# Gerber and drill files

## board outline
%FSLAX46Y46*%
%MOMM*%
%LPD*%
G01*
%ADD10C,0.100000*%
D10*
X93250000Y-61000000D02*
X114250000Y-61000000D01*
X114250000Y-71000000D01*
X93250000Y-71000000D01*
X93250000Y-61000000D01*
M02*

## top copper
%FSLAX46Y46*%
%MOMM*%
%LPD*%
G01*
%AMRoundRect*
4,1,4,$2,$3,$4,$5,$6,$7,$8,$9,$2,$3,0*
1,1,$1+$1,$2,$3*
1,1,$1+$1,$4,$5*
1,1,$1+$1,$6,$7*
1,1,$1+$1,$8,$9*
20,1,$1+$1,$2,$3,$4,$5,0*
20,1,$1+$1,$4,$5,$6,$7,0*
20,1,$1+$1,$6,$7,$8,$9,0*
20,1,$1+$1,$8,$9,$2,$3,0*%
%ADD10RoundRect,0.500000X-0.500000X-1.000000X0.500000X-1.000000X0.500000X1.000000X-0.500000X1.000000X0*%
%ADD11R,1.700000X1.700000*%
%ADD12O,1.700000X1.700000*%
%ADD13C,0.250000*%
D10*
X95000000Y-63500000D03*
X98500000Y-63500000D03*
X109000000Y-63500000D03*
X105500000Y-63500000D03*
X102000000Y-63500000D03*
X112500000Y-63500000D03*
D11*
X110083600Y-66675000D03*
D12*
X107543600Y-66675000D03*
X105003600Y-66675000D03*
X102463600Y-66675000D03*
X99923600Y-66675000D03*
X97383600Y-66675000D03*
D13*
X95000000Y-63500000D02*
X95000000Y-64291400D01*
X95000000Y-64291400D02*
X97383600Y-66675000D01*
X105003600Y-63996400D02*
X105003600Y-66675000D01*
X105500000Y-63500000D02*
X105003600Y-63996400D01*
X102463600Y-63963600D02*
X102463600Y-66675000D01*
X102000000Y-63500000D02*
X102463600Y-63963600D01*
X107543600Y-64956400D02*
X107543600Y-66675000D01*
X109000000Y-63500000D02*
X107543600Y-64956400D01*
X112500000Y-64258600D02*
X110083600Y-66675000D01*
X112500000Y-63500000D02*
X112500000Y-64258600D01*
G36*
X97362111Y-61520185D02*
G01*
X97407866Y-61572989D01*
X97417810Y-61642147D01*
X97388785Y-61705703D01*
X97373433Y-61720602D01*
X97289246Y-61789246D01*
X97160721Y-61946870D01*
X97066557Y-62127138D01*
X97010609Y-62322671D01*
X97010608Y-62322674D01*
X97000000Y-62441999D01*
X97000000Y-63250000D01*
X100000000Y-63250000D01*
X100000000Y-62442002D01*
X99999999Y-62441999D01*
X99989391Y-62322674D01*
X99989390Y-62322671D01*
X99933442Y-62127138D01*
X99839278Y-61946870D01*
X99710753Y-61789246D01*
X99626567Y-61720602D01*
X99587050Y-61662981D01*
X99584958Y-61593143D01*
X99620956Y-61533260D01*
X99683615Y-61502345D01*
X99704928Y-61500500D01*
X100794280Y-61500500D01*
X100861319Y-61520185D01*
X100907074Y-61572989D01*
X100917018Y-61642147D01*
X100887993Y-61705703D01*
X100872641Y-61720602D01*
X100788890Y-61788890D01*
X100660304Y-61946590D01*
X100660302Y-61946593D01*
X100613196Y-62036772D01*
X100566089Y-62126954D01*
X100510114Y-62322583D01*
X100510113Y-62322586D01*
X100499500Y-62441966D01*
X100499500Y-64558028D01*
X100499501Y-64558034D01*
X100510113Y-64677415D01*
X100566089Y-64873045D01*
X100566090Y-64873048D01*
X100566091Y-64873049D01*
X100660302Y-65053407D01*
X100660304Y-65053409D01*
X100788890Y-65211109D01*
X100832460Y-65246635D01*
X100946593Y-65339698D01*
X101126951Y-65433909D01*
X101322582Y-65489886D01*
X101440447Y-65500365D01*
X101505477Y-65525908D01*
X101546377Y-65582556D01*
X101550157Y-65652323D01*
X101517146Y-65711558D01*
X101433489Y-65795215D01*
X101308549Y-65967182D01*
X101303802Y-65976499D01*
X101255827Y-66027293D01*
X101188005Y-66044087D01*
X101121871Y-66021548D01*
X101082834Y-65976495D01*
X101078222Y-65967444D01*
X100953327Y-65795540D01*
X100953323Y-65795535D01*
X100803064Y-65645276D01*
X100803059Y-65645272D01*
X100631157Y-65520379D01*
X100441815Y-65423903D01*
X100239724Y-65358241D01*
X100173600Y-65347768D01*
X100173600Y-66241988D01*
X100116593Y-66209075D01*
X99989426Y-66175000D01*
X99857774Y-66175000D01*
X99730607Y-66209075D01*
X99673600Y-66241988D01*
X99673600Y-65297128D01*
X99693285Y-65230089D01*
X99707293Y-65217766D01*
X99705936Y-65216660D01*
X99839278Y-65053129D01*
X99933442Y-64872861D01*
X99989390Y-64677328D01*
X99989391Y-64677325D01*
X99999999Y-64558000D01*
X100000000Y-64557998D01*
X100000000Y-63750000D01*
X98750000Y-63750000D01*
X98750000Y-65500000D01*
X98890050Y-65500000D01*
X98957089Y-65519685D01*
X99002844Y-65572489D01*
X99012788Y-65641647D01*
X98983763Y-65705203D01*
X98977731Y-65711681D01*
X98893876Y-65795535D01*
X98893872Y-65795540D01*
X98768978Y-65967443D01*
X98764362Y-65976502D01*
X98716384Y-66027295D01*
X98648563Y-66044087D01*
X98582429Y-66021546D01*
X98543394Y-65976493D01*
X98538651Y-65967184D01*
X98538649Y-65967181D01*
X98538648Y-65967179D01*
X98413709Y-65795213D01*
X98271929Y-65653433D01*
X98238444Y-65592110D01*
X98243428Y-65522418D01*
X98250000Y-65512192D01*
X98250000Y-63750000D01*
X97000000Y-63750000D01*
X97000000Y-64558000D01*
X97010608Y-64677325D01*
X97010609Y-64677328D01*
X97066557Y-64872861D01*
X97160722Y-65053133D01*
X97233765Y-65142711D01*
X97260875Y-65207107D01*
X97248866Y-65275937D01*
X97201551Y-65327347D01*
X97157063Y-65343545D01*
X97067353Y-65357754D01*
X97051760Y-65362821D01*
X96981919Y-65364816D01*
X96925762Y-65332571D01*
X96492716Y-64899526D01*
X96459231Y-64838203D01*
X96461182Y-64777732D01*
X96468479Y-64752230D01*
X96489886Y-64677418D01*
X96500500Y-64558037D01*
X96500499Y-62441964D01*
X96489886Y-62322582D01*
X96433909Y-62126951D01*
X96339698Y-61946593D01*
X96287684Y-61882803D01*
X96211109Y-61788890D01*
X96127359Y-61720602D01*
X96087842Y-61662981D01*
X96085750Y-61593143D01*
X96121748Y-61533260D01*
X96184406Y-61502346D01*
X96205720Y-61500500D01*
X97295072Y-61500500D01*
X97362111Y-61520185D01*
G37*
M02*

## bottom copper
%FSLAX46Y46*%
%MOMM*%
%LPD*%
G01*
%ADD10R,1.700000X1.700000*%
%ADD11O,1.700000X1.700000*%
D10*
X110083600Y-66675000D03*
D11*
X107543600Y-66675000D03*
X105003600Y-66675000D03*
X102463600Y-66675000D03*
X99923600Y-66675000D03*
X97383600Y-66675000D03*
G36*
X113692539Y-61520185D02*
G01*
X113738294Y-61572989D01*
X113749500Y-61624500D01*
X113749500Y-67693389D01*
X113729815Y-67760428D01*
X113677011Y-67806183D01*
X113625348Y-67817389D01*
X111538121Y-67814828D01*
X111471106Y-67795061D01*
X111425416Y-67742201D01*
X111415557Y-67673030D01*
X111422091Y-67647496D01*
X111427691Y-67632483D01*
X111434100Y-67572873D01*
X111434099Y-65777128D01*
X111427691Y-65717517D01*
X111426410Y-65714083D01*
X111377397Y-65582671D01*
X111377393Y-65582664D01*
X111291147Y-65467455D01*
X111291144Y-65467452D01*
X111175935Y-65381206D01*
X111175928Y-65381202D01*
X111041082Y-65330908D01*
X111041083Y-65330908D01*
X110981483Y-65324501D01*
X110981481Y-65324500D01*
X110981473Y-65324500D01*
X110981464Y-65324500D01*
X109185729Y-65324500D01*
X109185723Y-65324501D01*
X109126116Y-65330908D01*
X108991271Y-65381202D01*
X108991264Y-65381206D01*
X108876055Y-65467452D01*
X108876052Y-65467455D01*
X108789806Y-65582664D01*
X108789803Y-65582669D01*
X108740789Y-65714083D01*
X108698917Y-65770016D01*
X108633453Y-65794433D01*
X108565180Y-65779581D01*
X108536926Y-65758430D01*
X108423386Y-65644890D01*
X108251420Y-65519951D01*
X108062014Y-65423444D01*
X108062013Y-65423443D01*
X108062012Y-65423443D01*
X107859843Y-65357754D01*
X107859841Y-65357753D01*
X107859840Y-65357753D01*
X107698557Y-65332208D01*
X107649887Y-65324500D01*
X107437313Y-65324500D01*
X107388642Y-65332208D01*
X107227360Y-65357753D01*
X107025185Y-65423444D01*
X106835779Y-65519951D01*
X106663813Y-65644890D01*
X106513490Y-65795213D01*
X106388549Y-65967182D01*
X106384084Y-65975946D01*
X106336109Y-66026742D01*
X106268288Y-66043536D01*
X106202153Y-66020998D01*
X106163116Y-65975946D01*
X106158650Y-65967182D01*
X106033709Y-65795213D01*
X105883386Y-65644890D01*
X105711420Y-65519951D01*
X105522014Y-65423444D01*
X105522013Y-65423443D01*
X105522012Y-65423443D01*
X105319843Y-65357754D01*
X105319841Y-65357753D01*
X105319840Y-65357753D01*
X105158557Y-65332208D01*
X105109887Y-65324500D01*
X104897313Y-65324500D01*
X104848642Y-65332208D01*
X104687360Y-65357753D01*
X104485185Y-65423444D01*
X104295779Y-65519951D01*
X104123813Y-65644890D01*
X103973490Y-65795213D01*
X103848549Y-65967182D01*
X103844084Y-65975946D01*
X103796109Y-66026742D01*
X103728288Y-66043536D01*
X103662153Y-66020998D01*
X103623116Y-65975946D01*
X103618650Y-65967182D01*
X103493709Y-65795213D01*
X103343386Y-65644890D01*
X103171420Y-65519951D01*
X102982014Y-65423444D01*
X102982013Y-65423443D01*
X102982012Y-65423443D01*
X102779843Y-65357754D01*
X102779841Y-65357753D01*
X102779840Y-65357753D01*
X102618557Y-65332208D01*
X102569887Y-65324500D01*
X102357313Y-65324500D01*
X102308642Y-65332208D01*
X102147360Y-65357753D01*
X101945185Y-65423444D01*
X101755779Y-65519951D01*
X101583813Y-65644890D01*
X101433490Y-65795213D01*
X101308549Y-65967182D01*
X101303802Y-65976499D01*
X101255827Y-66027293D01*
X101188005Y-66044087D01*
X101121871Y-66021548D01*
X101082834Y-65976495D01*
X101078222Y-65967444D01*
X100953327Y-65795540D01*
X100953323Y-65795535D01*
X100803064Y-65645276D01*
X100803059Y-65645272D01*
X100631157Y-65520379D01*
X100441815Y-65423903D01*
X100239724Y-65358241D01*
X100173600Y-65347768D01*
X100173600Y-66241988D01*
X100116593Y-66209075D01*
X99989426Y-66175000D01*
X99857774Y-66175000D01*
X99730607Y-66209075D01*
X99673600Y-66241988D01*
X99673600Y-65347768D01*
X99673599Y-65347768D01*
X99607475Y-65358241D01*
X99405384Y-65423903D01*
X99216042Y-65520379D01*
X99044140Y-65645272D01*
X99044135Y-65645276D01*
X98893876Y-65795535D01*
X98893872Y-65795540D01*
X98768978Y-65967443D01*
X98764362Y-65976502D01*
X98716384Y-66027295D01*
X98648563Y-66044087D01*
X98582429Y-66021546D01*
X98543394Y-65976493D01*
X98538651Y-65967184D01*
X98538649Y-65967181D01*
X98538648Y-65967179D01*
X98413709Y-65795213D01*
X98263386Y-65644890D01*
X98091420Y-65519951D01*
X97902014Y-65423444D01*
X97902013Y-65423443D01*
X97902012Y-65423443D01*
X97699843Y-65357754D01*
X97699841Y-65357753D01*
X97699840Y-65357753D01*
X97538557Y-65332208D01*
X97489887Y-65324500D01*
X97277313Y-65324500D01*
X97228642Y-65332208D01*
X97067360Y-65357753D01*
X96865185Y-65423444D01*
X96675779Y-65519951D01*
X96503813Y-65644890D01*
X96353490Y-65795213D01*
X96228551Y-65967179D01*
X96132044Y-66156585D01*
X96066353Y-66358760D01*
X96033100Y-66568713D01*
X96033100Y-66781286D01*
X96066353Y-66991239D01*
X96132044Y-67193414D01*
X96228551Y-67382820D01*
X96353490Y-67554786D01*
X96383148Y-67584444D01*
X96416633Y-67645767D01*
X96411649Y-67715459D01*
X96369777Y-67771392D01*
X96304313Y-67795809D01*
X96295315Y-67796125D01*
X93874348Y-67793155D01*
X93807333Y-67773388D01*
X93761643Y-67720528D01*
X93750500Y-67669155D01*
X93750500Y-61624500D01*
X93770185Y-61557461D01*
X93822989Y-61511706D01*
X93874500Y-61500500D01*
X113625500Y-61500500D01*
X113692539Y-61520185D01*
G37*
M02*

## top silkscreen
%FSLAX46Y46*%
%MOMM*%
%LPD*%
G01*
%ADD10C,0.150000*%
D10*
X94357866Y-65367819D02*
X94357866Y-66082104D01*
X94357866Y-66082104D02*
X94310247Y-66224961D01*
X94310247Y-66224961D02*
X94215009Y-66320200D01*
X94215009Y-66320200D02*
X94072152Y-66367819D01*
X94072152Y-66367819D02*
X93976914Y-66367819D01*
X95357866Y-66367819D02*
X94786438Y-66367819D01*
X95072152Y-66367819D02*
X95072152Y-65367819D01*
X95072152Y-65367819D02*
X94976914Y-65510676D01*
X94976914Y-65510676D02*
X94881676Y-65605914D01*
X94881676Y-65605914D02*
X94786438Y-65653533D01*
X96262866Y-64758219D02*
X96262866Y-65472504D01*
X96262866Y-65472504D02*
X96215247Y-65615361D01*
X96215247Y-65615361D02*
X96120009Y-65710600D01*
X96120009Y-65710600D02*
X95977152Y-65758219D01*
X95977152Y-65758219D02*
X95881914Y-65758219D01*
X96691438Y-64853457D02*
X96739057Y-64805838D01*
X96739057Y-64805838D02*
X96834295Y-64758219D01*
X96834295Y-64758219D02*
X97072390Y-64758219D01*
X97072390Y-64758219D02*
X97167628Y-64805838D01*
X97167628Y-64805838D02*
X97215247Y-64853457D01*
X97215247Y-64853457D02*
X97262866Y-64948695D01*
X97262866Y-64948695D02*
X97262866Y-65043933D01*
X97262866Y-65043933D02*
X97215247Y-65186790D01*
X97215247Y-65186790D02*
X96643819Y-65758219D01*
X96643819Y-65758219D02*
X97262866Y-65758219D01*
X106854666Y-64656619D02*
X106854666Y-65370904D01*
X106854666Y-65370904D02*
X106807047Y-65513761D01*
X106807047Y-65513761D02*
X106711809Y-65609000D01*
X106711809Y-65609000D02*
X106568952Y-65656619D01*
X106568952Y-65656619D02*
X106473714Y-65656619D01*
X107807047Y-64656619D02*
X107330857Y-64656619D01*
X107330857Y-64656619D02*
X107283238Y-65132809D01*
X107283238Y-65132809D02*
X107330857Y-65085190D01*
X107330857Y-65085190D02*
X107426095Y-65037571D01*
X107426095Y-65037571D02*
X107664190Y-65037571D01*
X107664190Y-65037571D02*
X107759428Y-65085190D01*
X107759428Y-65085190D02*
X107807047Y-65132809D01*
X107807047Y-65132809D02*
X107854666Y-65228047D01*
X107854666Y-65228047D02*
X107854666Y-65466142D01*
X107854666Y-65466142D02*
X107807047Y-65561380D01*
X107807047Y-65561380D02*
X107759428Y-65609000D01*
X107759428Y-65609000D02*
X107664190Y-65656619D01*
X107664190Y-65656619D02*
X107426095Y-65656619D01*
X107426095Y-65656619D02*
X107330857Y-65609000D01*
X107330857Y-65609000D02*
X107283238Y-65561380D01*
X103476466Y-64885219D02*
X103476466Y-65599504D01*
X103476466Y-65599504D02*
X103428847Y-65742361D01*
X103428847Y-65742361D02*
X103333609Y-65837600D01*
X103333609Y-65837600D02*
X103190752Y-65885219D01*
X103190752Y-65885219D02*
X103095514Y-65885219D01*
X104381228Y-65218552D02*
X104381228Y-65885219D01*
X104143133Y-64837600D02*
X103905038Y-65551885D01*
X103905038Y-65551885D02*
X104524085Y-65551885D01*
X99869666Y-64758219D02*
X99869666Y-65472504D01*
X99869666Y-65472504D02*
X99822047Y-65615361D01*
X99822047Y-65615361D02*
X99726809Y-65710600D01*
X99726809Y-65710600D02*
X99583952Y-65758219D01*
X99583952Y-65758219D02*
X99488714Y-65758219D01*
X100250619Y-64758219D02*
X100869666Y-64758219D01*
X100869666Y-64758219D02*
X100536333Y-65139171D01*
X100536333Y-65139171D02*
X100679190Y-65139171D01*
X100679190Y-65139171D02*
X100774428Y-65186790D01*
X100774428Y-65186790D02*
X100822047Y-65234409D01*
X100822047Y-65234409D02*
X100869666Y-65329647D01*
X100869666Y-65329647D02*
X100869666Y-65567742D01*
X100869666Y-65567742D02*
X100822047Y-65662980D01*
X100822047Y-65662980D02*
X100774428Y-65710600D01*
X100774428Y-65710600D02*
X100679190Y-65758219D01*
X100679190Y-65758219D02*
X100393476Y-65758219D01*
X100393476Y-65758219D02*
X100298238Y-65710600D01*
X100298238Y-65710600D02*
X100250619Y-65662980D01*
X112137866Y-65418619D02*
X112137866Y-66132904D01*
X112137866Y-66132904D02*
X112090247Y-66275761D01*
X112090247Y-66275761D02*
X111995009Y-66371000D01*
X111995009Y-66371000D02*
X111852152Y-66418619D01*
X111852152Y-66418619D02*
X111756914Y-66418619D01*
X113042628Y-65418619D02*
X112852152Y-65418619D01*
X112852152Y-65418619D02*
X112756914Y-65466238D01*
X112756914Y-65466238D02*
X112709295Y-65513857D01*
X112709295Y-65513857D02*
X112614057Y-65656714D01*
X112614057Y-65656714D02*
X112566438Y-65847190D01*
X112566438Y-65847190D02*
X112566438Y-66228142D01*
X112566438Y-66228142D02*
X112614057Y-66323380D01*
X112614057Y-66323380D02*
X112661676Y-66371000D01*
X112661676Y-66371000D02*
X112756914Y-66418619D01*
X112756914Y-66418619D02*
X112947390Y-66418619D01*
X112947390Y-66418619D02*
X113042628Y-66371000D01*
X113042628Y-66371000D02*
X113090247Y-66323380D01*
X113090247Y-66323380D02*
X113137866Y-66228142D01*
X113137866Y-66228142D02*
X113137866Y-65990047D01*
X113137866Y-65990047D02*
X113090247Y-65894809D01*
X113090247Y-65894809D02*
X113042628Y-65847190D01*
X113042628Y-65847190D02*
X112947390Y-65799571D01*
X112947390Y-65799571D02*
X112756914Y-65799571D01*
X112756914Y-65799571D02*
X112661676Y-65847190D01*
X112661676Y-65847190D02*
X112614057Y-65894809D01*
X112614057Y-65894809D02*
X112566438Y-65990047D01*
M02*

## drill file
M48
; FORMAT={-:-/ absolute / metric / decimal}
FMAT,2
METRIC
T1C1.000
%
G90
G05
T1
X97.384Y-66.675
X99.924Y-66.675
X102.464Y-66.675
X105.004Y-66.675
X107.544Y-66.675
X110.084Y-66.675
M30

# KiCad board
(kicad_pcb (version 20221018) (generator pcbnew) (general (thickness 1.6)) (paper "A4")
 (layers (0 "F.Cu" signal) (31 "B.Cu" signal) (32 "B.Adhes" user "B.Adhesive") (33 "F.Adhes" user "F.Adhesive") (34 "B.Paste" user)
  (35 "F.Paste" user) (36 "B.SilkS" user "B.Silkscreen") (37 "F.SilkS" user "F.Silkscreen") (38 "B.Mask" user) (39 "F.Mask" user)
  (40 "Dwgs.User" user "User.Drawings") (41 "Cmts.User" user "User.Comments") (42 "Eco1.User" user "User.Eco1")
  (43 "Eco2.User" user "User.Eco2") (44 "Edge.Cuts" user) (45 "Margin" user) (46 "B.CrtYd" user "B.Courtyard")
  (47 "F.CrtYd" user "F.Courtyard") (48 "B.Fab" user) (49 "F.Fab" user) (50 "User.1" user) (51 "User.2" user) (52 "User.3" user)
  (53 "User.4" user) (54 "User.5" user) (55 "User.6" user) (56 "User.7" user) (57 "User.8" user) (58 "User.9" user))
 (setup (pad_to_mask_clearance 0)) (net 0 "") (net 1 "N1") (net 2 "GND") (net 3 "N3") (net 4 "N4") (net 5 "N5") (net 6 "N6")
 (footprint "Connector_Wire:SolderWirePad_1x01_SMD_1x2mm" (layer "F.Cu") (at 95 63.5)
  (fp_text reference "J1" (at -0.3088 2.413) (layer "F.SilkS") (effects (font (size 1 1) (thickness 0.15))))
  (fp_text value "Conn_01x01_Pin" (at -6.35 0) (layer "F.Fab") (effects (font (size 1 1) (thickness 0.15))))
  (pad "1" smd roundrect (at 0 0) (size 2 3) (layers "F.Cu" "F.Paste" "F.Mask") (roundrect_rratio 0.25) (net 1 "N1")))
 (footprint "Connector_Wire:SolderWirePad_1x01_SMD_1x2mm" (layer "F.Cu") (at 98.5 63.5)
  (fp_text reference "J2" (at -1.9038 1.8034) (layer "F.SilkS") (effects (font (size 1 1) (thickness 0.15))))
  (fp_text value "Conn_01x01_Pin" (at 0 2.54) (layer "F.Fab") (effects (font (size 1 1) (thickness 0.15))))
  (pad "1" smd roundrect (at 0 0) (size 2 3) (layers "F.Cu" "F.Paste" "F.Mask") (roundrect_rratio 0.25) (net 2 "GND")))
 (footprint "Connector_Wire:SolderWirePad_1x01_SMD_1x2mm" (layer "F.Cu") (at 109 63.5)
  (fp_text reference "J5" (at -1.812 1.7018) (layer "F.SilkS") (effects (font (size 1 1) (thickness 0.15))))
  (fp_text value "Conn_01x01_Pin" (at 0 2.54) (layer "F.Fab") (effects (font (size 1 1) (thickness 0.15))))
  (pad "1" smd roundrect (at 0 0) (size 2 3) (layers "F.Cu" "F.Paste" "F.Mask") (roundrect_rratio 0.25) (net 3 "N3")))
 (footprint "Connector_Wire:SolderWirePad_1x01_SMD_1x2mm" (layer "F.Cu") (at 105.5 63.5)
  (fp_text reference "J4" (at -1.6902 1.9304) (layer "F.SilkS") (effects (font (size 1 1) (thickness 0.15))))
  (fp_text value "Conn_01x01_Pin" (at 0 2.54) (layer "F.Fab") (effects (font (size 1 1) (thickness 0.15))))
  (pad "1" smd roundrect (at 0 0) (size 2 3) (layers "F.Cu" "F.Paste" "F.Mask") (roundrect_rratio 0.25) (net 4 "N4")))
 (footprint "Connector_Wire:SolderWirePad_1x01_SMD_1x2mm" (layer "F.Cu") (at 102 63.5)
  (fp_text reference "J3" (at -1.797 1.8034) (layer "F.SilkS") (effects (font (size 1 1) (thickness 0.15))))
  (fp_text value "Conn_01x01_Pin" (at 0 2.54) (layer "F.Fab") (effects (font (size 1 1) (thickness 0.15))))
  (pad "1" smd roundrect (at 0 0) (size 2 3) (layers "F.Cu" "F.Paste" "F.Mask") (roundrect_rratio 0.25) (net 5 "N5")))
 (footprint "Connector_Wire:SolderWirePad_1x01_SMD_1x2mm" (layer "F.Cu") (at 112.5 63.5)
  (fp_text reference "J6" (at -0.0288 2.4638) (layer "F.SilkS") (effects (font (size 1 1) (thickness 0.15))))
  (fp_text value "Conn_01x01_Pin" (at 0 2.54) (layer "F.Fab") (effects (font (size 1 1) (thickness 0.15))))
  (pad "1" smd roundrect (at 0 0) (size 2 3) (layers "F.Cu" "F.Paste" "F.Mask") (roundrect_rratio 0.25) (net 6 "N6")))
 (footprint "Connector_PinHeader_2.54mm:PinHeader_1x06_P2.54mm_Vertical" (layer "B.Cu") (at 110.0836 66.675 90)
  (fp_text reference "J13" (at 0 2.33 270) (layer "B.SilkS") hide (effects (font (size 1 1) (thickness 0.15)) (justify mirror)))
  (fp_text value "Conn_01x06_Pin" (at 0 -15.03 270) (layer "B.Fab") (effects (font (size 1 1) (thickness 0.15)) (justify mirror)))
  (pad "1" thru_hole rect (at 0 0 90) (size 1.7 1.7) (drill 1) (layers "*.Cu" "*.Mask") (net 6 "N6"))
  (pad "2" thru_hole oval (at 0 -2.54 90) (size 1.7 1.7) (drill 1) (layers "*.Cu" "*.Mask") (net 3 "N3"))
  (pad "3" thru_hole oval (at 0 -5.08 90) (size 1.7 1.7) (drill 1) (layers "*.Cu" "*.Mask") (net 4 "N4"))
  (pad "4" thru_hole oval (at 0 -7.62 90) (size 1.7 1.7) (drill 1) (layers "*.Cu" "*.Mask") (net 5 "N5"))
  (pad "5" thru_hole oval (at 0 -10.16 90) (size 1.7 1.7) (drill 1) (layers "*.Cu" "*.Mask") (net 2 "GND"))
  (pad "6" thru_hole oval (at 0 -12.7 90) (size 1.7 1.7) (drill 1) (layers "*.Cu" "*.Mask") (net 1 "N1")))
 (gr_poly (pts (xy 93.25 61) (xy 114.25 61) (xy 114.25 71) (xy 93.25 71)) (stroke (width 0.1) (type solid)) (fill none) (layer "Edge.Cuts"))
 (segment (start 95 63.5) (end 95 64.2914) (width 0.25) (layer "F.Cu") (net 1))
 (segment (start 95 64.2914) (end 97.3836 66.675) (width 0.25) (layer "F.Cu") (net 1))
 (segment (start 105.0036 63.9964) (end 105.0036 66.675) (width 0.25) (layer "F.Cu") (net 4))
 (segment (start 105.5 63.5) (end 105.0036 63.9964) (width 0.25) (layer "F.Cu") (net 4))
 (segment (start 102.4636 63.9636) (end 102.4636 66.675) (width 0.25) (layer "F.Cu") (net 5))
 (segment (start 102 63.5) (end 102.4636 63.9636) (width 0.25) (layer "F.Cu") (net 5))
 (segment (start 107.5436 64.9564) (end 107.5436 66.675) (width 0.25) (layer "F.Cu") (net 3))
 (segment (start 109 63.5) (end 107.5436 64.9564) (width 0.25) (layer "F.Cu") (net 3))
 (segment (start 112.5 64.2586) (end 110.0836 66.675) (width 0.25) (layer "F.Cu") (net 6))
 (segment (start 112.5 63.5) (end 112.5 64.2586) (width 0.25) (layer "F.Cu") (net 6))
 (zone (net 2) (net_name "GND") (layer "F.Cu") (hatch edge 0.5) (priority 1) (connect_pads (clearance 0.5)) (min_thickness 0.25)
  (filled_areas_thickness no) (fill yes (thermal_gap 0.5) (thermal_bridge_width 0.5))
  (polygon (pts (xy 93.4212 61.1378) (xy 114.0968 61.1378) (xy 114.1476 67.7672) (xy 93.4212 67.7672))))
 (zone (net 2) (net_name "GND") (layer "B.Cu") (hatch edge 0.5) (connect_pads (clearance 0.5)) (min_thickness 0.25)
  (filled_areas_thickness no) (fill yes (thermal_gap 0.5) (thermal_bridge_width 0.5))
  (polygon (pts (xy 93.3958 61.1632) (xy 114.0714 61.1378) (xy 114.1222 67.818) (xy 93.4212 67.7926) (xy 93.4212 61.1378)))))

